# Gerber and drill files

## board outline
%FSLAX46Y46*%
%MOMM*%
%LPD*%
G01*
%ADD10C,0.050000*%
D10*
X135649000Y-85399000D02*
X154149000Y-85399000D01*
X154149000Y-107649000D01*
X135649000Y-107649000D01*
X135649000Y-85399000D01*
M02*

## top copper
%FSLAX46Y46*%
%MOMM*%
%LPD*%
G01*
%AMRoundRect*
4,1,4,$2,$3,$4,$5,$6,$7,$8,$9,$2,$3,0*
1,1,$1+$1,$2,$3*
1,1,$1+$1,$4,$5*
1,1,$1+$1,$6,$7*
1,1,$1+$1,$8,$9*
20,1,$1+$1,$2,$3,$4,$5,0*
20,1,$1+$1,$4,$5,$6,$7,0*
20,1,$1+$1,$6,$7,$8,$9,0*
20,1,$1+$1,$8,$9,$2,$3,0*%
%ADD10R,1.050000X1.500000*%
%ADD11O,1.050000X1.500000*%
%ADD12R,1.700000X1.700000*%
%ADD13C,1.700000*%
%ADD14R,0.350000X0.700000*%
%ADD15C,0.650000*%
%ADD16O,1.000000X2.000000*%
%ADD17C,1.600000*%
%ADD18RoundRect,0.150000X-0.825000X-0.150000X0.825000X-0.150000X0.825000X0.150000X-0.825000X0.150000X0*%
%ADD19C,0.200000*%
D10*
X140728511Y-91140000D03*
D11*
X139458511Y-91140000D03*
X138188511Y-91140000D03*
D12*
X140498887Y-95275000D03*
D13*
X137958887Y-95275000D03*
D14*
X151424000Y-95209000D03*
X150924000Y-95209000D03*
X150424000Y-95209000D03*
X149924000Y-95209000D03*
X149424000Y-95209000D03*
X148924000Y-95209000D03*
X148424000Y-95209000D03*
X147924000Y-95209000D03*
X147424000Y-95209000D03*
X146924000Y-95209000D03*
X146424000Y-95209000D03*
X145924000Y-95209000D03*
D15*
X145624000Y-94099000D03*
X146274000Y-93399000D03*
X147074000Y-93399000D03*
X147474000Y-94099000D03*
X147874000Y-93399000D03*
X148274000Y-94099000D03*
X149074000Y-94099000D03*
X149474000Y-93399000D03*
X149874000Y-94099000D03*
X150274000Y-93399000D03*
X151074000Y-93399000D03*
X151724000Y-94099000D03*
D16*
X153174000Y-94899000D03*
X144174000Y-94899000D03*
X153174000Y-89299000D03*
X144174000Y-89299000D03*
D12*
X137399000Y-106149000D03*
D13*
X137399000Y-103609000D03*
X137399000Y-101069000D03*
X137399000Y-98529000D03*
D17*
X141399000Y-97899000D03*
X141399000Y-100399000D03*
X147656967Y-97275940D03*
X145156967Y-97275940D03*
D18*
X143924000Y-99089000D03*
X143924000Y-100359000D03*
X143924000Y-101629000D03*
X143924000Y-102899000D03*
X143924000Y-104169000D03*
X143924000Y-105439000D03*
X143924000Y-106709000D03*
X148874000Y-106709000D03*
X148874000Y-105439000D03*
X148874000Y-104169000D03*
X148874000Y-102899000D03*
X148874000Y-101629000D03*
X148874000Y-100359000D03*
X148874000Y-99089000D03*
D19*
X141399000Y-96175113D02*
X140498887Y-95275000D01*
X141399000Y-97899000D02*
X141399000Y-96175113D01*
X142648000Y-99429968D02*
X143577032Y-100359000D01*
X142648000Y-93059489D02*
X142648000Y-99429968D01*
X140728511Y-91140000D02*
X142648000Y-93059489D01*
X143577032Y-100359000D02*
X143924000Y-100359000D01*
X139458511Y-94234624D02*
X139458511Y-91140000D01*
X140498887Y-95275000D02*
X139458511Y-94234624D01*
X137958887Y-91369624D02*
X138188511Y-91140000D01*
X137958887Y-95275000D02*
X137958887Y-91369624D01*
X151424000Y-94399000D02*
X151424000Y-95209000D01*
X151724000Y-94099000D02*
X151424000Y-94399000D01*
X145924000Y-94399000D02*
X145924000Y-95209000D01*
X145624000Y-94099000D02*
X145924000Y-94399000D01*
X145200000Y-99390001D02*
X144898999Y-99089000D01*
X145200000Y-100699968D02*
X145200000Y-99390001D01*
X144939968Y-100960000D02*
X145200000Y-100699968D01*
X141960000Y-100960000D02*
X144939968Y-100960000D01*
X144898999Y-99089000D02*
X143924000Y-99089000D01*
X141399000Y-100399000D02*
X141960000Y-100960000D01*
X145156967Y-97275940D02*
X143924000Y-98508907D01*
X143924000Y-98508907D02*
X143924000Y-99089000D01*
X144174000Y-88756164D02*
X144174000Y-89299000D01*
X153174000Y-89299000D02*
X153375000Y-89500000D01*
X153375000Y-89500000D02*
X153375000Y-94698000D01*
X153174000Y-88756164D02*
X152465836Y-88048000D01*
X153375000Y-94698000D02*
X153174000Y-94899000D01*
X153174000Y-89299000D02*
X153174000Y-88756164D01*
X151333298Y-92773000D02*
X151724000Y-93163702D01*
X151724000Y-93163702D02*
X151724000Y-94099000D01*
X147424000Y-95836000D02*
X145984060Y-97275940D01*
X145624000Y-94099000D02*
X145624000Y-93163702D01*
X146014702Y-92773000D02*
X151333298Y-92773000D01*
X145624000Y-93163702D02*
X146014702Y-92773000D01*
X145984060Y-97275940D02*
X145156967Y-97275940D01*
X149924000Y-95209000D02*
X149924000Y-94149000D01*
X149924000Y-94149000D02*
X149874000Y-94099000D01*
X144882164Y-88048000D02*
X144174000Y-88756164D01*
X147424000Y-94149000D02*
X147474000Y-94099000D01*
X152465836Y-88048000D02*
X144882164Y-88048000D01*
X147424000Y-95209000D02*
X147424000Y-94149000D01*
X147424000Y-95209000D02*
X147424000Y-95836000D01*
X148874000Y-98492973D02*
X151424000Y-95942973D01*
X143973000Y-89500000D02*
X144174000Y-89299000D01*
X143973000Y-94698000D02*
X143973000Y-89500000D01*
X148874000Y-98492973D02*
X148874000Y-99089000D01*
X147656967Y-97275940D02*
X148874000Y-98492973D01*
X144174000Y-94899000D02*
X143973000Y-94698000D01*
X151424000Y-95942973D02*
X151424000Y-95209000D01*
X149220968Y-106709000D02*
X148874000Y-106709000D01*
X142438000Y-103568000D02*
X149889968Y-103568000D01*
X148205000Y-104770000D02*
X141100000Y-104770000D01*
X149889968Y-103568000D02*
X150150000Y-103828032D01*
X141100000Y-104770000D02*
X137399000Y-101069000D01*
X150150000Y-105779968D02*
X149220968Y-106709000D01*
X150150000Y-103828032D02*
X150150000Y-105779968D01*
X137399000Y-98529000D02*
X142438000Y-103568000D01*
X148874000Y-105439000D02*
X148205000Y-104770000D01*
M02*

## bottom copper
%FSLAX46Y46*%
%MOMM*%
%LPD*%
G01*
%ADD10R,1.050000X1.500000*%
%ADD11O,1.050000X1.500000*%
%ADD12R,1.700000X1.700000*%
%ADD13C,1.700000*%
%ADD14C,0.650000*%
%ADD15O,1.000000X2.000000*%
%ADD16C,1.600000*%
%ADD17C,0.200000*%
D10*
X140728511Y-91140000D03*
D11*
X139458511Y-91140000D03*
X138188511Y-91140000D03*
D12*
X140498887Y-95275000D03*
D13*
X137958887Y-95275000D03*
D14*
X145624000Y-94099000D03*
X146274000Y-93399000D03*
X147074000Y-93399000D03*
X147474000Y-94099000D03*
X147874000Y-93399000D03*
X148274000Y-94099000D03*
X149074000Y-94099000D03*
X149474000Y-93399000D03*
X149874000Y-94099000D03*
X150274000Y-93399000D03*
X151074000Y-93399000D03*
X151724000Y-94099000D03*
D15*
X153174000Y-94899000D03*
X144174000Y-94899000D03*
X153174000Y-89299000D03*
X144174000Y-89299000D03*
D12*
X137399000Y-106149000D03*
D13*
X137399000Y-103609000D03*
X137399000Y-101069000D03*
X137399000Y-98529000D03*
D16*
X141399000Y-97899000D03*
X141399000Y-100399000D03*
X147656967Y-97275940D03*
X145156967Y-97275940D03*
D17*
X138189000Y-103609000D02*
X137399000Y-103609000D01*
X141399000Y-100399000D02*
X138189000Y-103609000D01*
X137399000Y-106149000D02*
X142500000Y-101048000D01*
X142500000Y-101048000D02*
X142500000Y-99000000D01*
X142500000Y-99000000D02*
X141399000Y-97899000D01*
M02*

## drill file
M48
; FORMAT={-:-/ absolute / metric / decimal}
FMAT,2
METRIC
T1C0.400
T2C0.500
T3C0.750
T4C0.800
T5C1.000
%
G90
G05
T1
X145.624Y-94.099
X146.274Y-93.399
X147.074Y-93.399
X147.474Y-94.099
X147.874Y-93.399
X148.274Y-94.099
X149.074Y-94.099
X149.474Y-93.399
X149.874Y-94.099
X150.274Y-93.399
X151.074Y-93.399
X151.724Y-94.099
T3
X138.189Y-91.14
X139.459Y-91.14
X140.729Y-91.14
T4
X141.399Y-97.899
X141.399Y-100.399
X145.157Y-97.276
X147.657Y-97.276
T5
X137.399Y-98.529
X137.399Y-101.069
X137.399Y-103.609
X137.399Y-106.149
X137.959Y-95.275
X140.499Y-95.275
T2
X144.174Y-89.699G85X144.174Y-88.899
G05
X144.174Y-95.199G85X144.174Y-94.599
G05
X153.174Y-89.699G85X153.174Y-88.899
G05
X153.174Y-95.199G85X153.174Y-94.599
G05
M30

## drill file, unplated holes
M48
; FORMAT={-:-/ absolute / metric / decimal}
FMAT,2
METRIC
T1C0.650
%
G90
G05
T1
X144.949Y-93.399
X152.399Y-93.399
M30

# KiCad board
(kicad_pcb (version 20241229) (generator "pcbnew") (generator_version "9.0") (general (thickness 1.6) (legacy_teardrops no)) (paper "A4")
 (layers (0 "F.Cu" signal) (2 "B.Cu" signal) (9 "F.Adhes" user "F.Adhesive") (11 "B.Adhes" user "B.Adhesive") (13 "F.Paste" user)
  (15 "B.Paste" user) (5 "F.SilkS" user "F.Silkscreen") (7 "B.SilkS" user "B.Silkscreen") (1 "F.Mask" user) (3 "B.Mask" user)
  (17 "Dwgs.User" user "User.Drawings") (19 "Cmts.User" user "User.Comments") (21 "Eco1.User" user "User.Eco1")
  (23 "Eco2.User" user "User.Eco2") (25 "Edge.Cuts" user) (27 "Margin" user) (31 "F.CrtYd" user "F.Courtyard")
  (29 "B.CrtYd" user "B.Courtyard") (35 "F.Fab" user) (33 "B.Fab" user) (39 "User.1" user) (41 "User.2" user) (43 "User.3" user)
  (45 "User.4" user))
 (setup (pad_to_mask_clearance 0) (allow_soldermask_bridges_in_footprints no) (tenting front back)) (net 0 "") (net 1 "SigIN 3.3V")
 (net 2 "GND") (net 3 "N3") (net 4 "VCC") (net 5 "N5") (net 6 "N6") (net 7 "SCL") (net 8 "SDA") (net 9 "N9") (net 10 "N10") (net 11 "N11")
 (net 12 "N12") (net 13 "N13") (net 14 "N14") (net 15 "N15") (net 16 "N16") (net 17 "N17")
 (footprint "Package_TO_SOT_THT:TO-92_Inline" (layer "F.Cu") (at 140.728511 91.14 180)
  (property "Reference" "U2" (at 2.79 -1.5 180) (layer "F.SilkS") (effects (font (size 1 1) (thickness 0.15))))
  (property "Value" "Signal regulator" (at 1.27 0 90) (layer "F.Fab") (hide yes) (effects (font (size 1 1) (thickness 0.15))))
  (pad "1" thru_hole rect (at 0 0 180) (size 1.05 1.5) (drill 0.75) (layers "*.Cu" "*.Mask") (remove_unused_layers no) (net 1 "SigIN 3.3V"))
  (pad "2" thru_hole oval (at 1.27 0 180) (size 1.05 1.5) (drill 0.75) (layers "*.Cu" "*.Mask") (remove_unused_layers no) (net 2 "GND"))
  (pad "3" thru_hole oval (at 2.54 0 180) (size 1.05 1.5) (drill 0.75) (layers "*.Cu" "*.Mask") (remove_unused_layers no) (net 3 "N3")))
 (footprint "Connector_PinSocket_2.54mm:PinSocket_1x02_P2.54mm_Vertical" (layer "F.Cu") (at 140.498887 95.275 -90)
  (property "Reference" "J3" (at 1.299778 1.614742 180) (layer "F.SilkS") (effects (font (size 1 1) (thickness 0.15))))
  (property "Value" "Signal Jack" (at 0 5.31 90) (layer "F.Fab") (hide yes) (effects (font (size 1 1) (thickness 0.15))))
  (pad "1" thru_hole rect (at 0 0 270) (size 1.7 1.7) (drill 1) (layers "*.Cu" "*.Mask") (remove_unused_layers no) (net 2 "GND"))
  (pad "2" thru_hole circle (at 0 2.54 270) (size 1.7 1.7) (drill 1) (layers "*.Cu" "*.Mask") (remove_unused_layers no) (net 3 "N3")))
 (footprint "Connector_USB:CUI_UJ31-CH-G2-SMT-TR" (layer "F.Cu") (at 151.424 95.209 180)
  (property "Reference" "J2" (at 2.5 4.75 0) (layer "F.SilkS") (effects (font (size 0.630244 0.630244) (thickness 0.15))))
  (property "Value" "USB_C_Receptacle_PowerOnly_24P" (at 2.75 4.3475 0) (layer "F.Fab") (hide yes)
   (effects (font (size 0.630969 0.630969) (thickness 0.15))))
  (pad "" np_thru_hole circle (at -0.975 1.81 180) (size 0.65 0.65) (drill 0.65) (layers "*.Cu" "*.Mask"))
  (pad "" np_thru_hole circle (at 6.475 1.81 180) (size 0.65 0.65) (drill 0.65) (layers "*.Cu" "*.Mask"))
  (pad "A1" smd rect (at 0 0 180) (size 0.35 0.7) (layers "F.Cu" "F.Mask" "F.Paste") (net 2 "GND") (solder_mask_margin 0.102))
  (pad "A2" smd rect (at 0.5 0 180) (size 0.35 0.7) (layers "F.Cu" "F.Mask" "F.Paste") (solder_mask_margin 0.102))
  (pad "A3" smd rect (at 1 0 180) (size 0.35 0.7) (layers "F.Cu" "F.Mask" "F.Paste") (solder_mask_margin 0.102))
  (pad "A4" smd rect (at 1.5 0 180) (size 0.35 0.7) (layers "F.Cu" "F.Mask" "F.Paste") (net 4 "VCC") (solder_mask_margin 0.102))
  (pad "A5" smd rect (at 2 0 180) (size 0.35 0.7) (layers "F.Cu" "F.Mask" "F.Paste") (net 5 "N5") (solder_mask_margin 0.102))
  (pad "A6" smd rect (at 2.5 0 180) (size 0.35 0.7) (layers "F.Cu" "F.Mask" "F.Paste") (solder_mask_margin 0.102))
  (pad "A7" smd rect (at 3 0 180) (size 0.35 0.7) (layers "F.Cu" "F.Mask" "F.Paste") (solder_mask_margin 0.102))
  (pad "A8" smd rect (at 3.5 0 180) (size 0.35 0.7) (layers "F.Cu" "F.Mask" "F.Paste") (solder_mask_margin 0.102))
  (pad "A9" smd rect (at 4 0 180) (size 0.35 0.7) (layers "F.Cu" "F.Mask" "F.Paste") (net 4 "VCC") (solder_mask_margin 0.102))
  (pad "A10" smd rect (at 4.5 0 180) (size 0.35 0.7) (layers "F.Cu" "F.Mask" "F.Paste") (solder_mask_margin 0.102))
  (pad "A11" smd rect (at 5 0 180) (size 0.35 0.7) (layers "F.Cu" "F.Mask" "F.Paste") (solder_mask_margin 0.102))
  (pad "A12" smd rect (at 5.5 0 180) (size 0.35 0.7) (layers "F.Cu" "F.Mask" "F.Paste") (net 2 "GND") (solder_mask_margin 0.102))
  (pad "B1" thru_hole circle (at 5.8 1.11 180) (size 0.65 0.65) (drill 0.4) (layers "*.Cu" "*.Mask") (remove_unused_layers no) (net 2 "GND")
   (solder_mask_margin 0.102))
  (pad "B2" thru_hole circle (at 5.15 1.81 180) (size 0.65 0.65) (drill 0.4) (layers "*.Cu" "*.Mask") (remove_unused_layers no)
   (solder_mask_margin 0.102))
  (pad "B3" thru_hole circle (at 4.35 1.81 180) (size 0.65 0.65) (drill 0.4) (layers "*.Cu" "*.Mask") (remove_unused_layers no)
   (solder_mask_margin 0.102))
  (pad "B4" thru_hole circle (at 3.95 1.11 180) (size 0.65 0.65) (drill 0.4) (layers "*.Cu" "*.Mask") (remove_unused_layers no)
   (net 4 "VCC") (solder_mask_margin 0.102))
  (pad "B5" thru_hole circle (at 3.55 1.81 180) (size 0.65 0.65) (drill 0.4) (layers "*.Cu" "*.Mask") (remove_unused_layers no) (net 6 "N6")
   (solder_mask_margin 0.102))
  (pad "B6" thru_hole circle (at 3.15 1.11 180) (size 0.65 0.65) (drill 0.4) (layers "*.Cu" "*.Mask") (remove_unused_layers no)
   (solder_mask_margin 0.102))
  (pad "B7" thru_hole circle (at 2.35 1.11 180) (size 0.65 0.65) (drill 0.4) (layers "*.Cu" "*.Mask") (remove_unused_layers no)
   (solder_mask_margin 0.102))
  (pad "B8" thru_hole circle (at 1.95 1.81 180) (size 0.65 0.65) (drill 0.4) (layers "*.Cu" "*.Mask") (remove_unused_layers no)
   (solder_mask_margin 0.102))
  (pad "B9" thru_hole circle (at 1.55 1.11 180) (size 0.65 0.65) (drill 0.4) (layers "*.Cu" "*.Mask") (remove_unused_layers no)
   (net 4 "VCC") (solder_mask_margin 0.102))
  (pad "B10" thru_hole circle (at 1.15 1.81 180) (size 0.65 0.65) (drill 0.4) (layers "*.Cu" "*.Mask") (remove_unused_layers no)
   (solder_mask_margin 0.102))
  (pad "B11" thru_hole circle (at 0.35 1.81 180) (size 0.65 0.65) (drill 0.4) (layers "*.Cu" "*.Mask") (remove_unused_layers no)
   (solder_mask_margin 0.102))
  (pad "B12" thru_hole circle (at -0.3 1.11 180) (size 0.65 0.65) (drill 0.4) (layers "*.Cu" "*.Mask") (remove_unused_layers no)
   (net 2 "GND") (solder_mask_margin 0.102))
  (pad "SH1" thru_hole oval (at -1.75 0.31 180) (size 1 2) (drill oval 0.5 1.1) (layers "*.Cu" "*.Mask") (remove_unused_layers no)
   (solder_mask_margin 0.102))
  (pad "SH2" thru_hole oval (at 7.25 0.31 180) (size 1 2) (drill oval 0.5 1.1) (layers "*.Cu" "*.Mask") (remove_unused_layers no)
   (solder_mask_margin 0.102))
  (pad "SH3" thru_hole oval (at -1.75 5.91 180) (size 1 2) (drill oval 0.5 1.3) (layers "*.Cu" "*.Mask") (remove_unused_layers no)
   (solder_mask_margin 0.102))
  (pad "SH4" thru_hole oval (at 7.25 5.91 180) (size 1 2) (drill oval 0.5 1.3) (layers "*.Cu" "*.Mask") (remove_unused_layers no)
   (solder_mask_margin 0.102))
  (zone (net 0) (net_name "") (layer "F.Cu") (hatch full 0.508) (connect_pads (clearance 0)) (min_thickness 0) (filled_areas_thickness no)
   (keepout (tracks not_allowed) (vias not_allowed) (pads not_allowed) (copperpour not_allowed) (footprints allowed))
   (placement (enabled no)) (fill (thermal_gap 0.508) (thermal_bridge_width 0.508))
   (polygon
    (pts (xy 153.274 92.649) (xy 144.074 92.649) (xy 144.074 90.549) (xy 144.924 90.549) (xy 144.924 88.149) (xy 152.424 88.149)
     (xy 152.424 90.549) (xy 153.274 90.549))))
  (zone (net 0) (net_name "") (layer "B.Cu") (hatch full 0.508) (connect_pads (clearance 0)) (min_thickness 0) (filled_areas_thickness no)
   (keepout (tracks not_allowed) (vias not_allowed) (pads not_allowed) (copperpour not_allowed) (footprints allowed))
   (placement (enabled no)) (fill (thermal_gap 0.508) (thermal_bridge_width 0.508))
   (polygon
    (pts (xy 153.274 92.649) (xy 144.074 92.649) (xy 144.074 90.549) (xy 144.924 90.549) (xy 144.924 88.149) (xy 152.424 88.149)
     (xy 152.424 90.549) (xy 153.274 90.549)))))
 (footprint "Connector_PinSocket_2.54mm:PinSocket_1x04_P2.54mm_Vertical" (layer "F.Cu") (at 137.399 106.149 180)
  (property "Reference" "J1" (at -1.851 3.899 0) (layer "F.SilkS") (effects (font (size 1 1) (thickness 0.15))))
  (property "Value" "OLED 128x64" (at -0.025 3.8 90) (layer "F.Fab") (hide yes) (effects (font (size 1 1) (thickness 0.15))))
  (pad "1" thru_hole rect (at 0 0 180) (size 1.7 1.7) (drill 1) (layers "*.Cu" "*.Mask") (remove_unused_layers no) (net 2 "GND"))
  (pad "2" thru_hole circle (at 0 2.54 180) (size 1.7 1.7) (drill 1) (layers "*.Cu" "*.Mask") (remove_unused_layers no) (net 4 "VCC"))
  (pad "3" thru_hole circle (at 0 5.08 180) (size 1.7 1.7) (drill 1) (layers "*.Cu" "*.Mask") (remove_unused_layers no) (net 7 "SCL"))
  (pad "4" thru_hole circle (at 0 7.62 180) (size 1.7 1.7) (drill 1) (layers "*.Cu" "*.Mask") (remove_unused_layers no) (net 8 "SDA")))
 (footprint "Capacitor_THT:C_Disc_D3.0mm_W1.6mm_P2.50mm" (layer "F.Cu") (at 141.399 100.399 90)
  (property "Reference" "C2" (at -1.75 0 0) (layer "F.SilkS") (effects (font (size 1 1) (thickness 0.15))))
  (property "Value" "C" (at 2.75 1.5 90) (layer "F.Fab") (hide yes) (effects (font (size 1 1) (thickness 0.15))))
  (pad "1" thru_hole circle (at 0 0 90) (size 1.6 1.6) (drill 0.8) (layers "*.Cu" "*.Mask") (remove_unused_layers no) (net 4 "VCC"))
  (pad "2" thru_hole circle (at 2.5 0 90) (size 1.6 1.6) (drill 0.8) (layers "*.Cu" "*.Mask") (remove_unused_layers no) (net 2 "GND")))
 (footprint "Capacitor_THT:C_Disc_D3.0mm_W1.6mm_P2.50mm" (layer "F.Cu") (at 147.656967 97.27594 180)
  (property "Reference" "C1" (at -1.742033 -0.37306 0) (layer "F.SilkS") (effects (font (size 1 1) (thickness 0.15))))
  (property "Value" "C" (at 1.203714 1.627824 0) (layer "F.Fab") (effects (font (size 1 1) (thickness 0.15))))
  (pad "1" thru_hole circle (at 0 0 180) (size 1.6 1.6) (drill 0.8) (layers "*.Cu" "*.Mask") (remove_unused_layers no) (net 2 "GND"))
  (pad "2" thru_hole circle (at 2.5 0 180) (size 1.6 1.6) (drill 0.8) (layers "*.Cu" "*.Mask") (remove_unused_layers no) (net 4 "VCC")))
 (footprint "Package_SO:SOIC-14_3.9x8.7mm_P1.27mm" (layer "F.Cu") (at 146.399 102.899)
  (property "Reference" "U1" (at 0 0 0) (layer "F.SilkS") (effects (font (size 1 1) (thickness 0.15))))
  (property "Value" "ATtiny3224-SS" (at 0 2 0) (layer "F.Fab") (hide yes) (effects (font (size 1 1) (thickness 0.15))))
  (pad "1" smd roundrect (at -2.475 -3.81) (size 1.95 0.6) (layers "F.Cu" "F.Mask" "F.Paste") (roundrect_rratio 0.25) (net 4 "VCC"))
  (pad "2" smd roundrect (at -2.475 -2.54) (size 1.95 0.6) (layers "F.Cu" "F.Mask" "F.Paste") (roundrect_rratio 0.25) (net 1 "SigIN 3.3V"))
  (pad "3" smd roundrect (at -2.475 -1.27) (size 1.95 0.6) (layers "F.Cu" "F.Mask" "F.Paste") (roundrect_rratio 0.25) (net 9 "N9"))
  (pad "4" smd roundrect (at -2.475 0) (size 1.95 0.6) (layers "F.Cu" "F.Mask" "F.Paste") (roundrect_rratio 0.25) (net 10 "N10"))
  (pad "5" smd roundrect (at -2.475 1.27) (size 1.95 0.6) (layers "F.Cu" "F.Mask" "F.Paste") (roundrect_rratio 0.25) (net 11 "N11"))
  (pad "6" smd roundrect (at -2.475 2.54) (size 1.95 0.6) (layers "F.Cu" "F.Mask" "F.Paste") (roundrect_rratio 0.25) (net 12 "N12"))
  (pad "7" smd roundrect (at -2.475 3.81) (size 1.95 0.6) (layers "F.Cu" "F.Mask" "F.Paste") (roundrect_rratio 0.25) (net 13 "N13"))
  (pad "8" smd roundrect (at 2.475 3.81) (size 1.95 0.6) (layers "F.Cu" "F.Mask" "F.Paste") (roundrect_rratio 0.25) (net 8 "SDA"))
  (pad "9" smd roundrect (at 2.475 2.54) (size 1.95 0.6) (layers "F.Cu" "F.Mask" "F.Paste") (roundrect_rratio 0.25) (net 7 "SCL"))
  (pad "10" smd roundrect (at 2.475 1.27) (size 1.95 0.6) (layers "F.Cu" "F.Mask" "F.Paste") (roundrect_rratio 0.25) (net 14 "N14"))
  (pad "11" smd roundrect (at 2.475 0) (size 1.95 0.6) (layers "F.Cu" "F.Mask" "F.Paste") (roundrect_rratio 0.25) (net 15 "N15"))
  (pad "12" smd roundrect (at 2.475 -1.27) (size 1.95 0.6) (layers "F.Cu" "F.Mask" "F.Paste") (roundrect_rratio 0.25) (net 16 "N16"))
  (pad "13" smd roundrect (at 2.475 -2.54) (size 1.95 0.6) (layers "F.Cu" "F.Mask" "F.Paste") (roundrect_rratio 0.25) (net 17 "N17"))
  (pad "14" smd roundrect (at 2.475 -3.81) (size 1.95 0.6) (layers "F.Cu" "F.Mask" "F.Paste") (roundrect_rratio 0.25) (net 2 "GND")))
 (gr_rect (start 135.649 85.399) (end 154.149 107.649) (stroke (width 0.05) (type default)) (fill no) (layer "Edge.Cuts"))
 (segment (start 153.375 94.698) (end 153.174 94.899) (width 0.2) (layer "F.Cu") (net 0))
 (segment (start 153.375 89.5) (end 153.375 94.698) (width 0.2) (layer "F.Cu") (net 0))
 (segment (start 144.174 88.756164) (end 144.174 89.299) (width 0.2) (layer "F.Cu") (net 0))
 (segment (start 152.465836 88.048) (end 144.882164 88.048) (width 0.2) (layer "F.Cu") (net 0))
 (segment (start 144.174 94.899) (end 143.973 94.698) (width 0.2) (layer "F.Cu") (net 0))
 (segment (start 153.174 89.299) (end 153.375 89.5) (width 0.2) (layer "F.Cu") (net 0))
 (segment (start 143.973 94.698) (end 143.973 89.5) (width 0.2) (layer "F.Cu") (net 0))
 (segment (start 153.174 88.756164) (end 152.465836 88.048) (width 0.2) (layer "F.Cu") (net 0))
 (segment (start 143.973 89.5) (end 144.174 89.299) (width 0.2) (layer "F.Cu") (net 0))
 (segment (start 144.882164 88.048) (end 144.174 88.756164) (width 0.2) (layer "F.Cu") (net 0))
 (segment (start 153.174 89.299) (end 153.174 88.756164) (width 0.2) (layer "F.Cu") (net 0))
 (segment (start 148.205 104.77) (end 141.1 104.77) (width 0.2) (layer "F.Cu") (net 7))
 (segment (start 148.874 105.439) (end 148.205 104.77) (width 0.2) (layer "F.Cu") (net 7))
 (segment (start 141.1 104.77) (end 137.399 101.069) (width 0.2) (layer "F.Cu") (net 7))
 (segment (start 149.220968 106.709) (end 148.874 106.709) (width 0.2) (layer "F.Cu") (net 8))
 (segment (start 137.399 98.529) (end 142.438 103.568) (width 0.2) (layer "F.Cu") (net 8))
 (segment (start 150.15 105.779968) (end 149.220968 106.709) (width 0.2) (layer "F.Cu") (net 8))
 (segment (start 150.15 103.828032) (end 150.15 105.779968) (width 0.2) (layer "F.Cu") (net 8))
 (segment (start 149.889968 103.568) (end 150.15 103.828032) (width 0.2) (layer "F.Cu") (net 8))
 (segment (start 142.438 103.568) (end 149.889968 103.568) (width 0.2) (layer "F.Cu") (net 8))
 (segment (start 147.424 95.209) (end 147.424 95.836) (width 0.2) (layer "F.Cu") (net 4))
 (segment (start 147.424 95.836) (end 145.98406 97.27594) (width 0.2) (layer "F.Cu") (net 4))
 (segment (start 141.399 100.399) (end 141.96 100.96) (width 0.2) (layer "F.Cu") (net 4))
 (segment (start 145.156967 97.27594) (end 143.924 98.508907) (width 0.2) (layer "F.Cu") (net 4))
 (segment (start 144.939968 100.96) (end 145.2 100.699968) (width 0.2) (layer "F.Cu") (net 4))
 (segment (start 141.96 100.96) (end 144.939968 100.96) (width 0.2) (layer "F.Cu") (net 4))
 (segment (start 145.98406 97.27594) (end 145.156967 97.27594) (width 0.2) (layer "F.Cu") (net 4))
 (segment (start 145.2 99.390001) (end 144.898999 99.089) (width 0.2) (layer "F.Cu") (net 4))
 (segment (start 149.924 95.209) (end 149.924 94.149) (width 0.2) (layer "F.Cu") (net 4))
 (segment (start 147.424 95.209) (end 147.424 94.149) (width 0.2) (layer "F.Cu") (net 4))
 (segment (start 143.924 98.508907) (end 143.924 99.089) (width 0.2) (layer "F.Cu") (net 4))
 (segment (start 147.424 94.149) (end 147.474 94.099) (width 0.2) (layer "F.Cu") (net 4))
 (segment (start 144.898999 99.089) (end 143.924 99.089) (width 0.2) (layer "F.Cu") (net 4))
 (segment (start 145.2 100.699968) (end 145.2 99.390001) (width 0.2) (layer "F.Cu") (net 4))
 (segment (start 149.924 94.149) (end 149.874 94.099) (width 0.2) (layer "F.Cu") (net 4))
 (segment (start 138.189 103.609) (end 137.399 103.609) (width 0.2) (layer "B.Cu") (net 4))
 (segment (start 141.399 100.399) (end 138.189 103.609) (width 0.2) (layer "B.Cu") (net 4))
 (segment (start 151.424 95.942973) (end 151.424 95.209) (width 0.2) (layer "F.Cu") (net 2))
 (segment (start 141.399 96.175113) (end 140.498887 95.275) (width 0.2) (layer "F.Cu") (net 2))
 (segment (start 151.333298 92.773) (end 151.724 93.163702) (width 0.2) (layer "F.Cu") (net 2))
 (segment (start 139.458511 94.234624) (end 139.458511 91.14) (width 0.2) (layer "F.Cu") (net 2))
 (segment (start 140.498887 95.275) (end 139.458511 94.234624) (width 0.2) (layer "F.Cu") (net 2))
 (segment (start 145.924 94.399) (end 145.924 95.209) (width 0.2) (layer "F.Cu") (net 2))
 (segment (start 151.424 94.399) (end 151.424 95.209) (width 0.2) (layer "F.Cu") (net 2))
 (segment (start 147.656967 97.27594) (end 148.874 98.492973) (width 0.2) (layer "F.Cu") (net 2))
 (segment (start 145.624 94.099) (end 145.924 94.399) (width 0.2) (layer "F.Cu") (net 2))
 (segment (start 148.874 98.492973) (end 151.424 95.942973) (width 0.2) (layer "F.Cu") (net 2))
 (segment (start 146.014702 92.773) (end 151.333298 92.773) (width 0.2) (layer "F.Cu") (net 2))
 (segment (start 141.399 97.899) (end 141.399 96.175113) (width 0.2) (layer "F.Cu") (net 2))
 (segment (start 148.874 98.492973) (end 148.874 99.089) (width 0.2) (layer "F.Cu") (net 2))
 (segment (start 151.724 93.163702) (end 151.724 94.099) (width 0.2) (layer "F.Cu") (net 2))
 (segment (start 145.624 94.099) (end 145.624 93.163702) (width 0.2) (layer "F.Cu") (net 2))
 (segment (start 151.724 94.099) (end 151.424 94.399) (width 0.2) (layer "F.Cu") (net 2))
 (segment (start 145.624 93.163702) (end 146.014702 92.773) (width 0.2) (layer "F.Cu") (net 2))
 (segment (start 142.5 99) (end 141.399 97.899) (width 0.2) (layer "B.Cu") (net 2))
 (segment (start 142.5 101.048) (end 142.5 99) (width 0.2) (layer "B.Cu") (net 2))
 (segment (start 137.399 106.149) (end 142.5 101.048) (width 0.2) (layer "B.Cu") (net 2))
 (segment (start 143.577032 100.359) (end 143.924 100.359) (width 0.2) (layer "F.Cu") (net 1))
 (segment (start 142.648 99.429968) (end 143.577032 100.359) (width 0.2) (layer "F.Cu") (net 1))
 (segment (start 142.648 93.059489) (end 142.648 99.429968) (width 0.2) (layer "F.Cu") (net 1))
 (segment (start 140.728511 91.14) (end 142.648 93.059489) (width 0.2) (layer "F.Cu") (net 1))
 (segment (start 137.958887 91.369624) (end 138.188511 91.14) (width 0.2) (layer "F.Cu") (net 3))
 (segment (start 137.958887 95.275) (end 137.958887 91.369624) (width 0.2) (layer "F.Cu") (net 3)))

